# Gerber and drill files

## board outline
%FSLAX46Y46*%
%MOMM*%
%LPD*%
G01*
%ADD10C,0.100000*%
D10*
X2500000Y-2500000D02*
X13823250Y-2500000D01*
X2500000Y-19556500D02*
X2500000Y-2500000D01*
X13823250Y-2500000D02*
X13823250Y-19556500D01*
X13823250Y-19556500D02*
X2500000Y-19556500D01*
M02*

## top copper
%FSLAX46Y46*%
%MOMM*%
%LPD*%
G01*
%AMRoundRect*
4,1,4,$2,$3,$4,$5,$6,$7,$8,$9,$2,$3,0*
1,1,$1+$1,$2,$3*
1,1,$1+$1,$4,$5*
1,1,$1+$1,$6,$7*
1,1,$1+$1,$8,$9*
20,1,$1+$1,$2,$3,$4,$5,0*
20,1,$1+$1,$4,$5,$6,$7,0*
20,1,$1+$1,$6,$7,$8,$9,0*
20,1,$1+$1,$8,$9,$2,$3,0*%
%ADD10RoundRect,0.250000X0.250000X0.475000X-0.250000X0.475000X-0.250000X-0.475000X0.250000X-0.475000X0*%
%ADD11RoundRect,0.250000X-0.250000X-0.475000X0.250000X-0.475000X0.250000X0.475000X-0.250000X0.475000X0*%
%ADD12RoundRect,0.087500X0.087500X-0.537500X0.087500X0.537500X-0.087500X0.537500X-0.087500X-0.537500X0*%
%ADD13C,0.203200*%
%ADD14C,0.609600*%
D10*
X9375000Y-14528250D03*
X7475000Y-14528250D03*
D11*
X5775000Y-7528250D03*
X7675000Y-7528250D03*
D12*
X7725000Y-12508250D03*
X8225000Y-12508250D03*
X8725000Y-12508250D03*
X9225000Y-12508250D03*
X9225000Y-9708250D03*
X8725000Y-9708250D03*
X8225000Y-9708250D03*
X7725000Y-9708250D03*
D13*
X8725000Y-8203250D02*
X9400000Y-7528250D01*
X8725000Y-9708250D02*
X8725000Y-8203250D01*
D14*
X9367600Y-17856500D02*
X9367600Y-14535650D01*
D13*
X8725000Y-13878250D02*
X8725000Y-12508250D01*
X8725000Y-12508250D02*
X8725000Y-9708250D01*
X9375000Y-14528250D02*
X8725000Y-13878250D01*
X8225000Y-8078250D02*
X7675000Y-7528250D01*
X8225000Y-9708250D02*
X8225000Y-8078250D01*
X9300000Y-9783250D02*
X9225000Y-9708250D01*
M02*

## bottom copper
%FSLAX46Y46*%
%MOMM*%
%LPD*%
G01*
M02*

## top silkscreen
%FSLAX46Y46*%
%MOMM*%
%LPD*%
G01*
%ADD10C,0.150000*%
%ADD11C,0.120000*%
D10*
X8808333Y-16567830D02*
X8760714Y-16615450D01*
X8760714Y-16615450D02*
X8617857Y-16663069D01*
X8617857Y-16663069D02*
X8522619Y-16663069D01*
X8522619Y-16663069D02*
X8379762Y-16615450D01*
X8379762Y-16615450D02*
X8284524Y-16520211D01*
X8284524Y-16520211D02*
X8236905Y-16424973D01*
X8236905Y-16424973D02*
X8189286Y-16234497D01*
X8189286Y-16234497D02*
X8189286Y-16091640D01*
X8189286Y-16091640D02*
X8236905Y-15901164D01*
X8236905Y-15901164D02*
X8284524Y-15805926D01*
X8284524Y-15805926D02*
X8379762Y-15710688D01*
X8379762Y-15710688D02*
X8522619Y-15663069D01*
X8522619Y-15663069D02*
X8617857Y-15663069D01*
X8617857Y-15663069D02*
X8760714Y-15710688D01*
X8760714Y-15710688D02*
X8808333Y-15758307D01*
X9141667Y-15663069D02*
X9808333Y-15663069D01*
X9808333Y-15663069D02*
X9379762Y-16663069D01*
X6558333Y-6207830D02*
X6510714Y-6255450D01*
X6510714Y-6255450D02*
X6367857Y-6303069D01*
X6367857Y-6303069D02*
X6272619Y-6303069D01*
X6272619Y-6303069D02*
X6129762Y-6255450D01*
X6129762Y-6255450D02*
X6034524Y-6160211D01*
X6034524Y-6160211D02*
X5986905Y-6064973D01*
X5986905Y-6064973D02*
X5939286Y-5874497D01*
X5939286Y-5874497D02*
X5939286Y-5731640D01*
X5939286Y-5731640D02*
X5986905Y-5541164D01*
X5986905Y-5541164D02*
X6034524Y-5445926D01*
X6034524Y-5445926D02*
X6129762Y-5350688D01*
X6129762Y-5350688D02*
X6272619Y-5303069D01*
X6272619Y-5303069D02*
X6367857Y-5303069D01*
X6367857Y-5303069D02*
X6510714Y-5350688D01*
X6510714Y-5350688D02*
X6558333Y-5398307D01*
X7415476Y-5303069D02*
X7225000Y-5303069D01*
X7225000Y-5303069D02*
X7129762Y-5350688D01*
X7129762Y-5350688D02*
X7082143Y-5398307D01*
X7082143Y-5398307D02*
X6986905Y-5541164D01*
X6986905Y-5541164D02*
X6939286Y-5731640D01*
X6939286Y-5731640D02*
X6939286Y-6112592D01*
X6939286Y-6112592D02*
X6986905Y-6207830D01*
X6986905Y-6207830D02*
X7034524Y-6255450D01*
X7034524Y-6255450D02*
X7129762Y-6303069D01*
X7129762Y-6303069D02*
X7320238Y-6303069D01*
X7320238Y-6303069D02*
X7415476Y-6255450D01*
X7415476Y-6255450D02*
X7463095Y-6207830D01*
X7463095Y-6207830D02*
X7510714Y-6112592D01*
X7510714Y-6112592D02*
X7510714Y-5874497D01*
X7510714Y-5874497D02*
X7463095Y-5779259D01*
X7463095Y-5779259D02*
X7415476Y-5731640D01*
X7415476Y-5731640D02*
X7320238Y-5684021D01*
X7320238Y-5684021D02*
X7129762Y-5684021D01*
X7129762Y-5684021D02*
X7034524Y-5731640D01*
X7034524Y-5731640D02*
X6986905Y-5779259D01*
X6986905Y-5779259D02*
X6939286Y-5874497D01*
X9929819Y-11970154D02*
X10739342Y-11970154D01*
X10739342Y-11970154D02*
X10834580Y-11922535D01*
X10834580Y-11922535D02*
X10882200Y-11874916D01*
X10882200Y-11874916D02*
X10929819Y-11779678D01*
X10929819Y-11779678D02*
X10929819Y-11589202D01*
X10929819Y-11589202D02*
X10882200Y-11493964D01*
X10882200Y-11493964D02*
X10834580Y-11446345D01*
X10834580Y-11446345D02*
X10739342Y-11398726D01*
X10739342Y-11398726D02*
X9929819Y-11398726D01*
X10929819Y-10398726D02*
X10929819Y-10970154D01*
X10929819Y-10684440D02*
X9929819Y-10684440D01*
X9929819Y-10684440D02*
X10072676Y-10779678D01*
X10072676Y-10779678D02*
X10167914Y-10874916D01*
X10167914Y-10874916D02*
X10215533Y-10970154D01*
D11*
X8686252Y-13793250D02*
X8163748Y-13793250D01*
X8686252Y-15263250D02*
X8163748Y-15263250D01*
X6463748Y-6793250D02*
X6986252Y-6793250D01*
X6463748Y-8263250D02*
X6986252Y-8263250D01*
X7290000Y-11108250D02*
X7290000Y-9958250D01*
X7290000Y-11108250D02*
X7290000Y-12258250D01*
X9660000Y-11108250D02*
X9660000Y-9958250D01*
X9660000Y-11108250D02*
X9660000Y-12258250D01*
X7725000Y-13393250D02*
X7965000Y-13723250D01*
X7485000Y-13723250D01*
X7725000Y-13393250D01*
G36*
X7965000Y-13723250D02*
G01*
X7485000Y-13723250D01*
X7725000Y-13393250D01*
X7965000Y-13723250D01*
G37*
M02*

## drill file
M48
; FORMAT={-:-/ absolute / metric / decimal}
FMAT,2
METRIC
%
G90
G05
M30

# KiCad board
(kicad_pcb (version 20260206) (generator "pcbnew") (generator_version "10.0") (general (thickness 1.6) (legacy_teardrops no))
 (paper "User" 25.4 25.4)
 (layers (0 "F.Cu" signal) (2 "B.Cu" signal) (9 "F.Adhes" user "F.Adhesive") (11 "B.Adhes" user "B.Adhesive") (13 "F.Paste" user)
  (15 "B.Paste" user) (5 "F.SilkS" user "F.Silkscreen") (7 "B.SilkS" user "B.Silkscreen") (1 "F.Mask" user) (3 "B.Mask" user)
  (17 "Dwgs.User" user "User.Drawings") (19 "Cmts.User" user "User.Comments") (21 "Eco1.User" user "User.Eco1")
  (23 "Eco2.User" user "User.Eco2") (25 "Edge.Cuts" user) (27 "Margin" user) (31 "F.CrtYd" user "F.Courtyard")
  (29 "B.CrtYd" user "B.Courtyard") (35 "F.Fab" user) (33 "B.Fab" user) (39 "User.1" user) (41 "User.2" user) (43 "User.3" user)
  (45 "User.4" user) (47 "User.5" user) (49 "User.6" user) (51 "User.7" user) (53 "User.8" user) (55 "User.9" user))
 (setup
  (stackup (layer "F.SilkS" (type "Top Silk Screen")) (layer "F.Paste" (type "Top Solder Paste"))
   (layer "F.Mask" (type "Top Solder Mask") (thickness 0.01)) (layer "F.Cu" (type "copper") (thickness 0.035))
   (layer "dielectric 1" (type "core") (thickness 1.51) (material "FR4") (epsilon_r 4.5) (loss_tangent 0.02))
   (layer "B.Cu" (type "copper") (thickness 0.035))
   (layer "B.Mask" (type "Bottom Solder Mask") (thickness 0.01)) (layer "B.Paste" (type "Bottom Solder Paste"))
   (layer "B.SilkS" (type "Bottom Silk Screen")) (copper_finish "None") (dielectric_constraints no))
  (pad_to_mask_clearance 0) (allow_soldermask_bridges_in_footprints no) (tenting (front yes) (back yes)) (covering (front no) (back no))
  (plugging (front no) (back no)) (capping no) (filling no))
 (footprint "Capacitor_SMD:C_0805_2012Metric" (layer "F.Cu") (at 8.425 14.52825 180)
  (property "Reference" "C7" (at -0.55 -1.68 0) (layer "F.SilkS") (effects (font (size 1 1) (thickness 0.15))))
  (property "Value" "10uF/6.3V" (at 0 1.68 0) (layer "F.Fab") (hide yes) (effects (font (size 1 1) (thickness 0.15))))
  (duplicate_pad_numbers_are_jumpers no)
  (fp_line (start -0.261252 0.735) (end 0.261252 0.735) (stroke (width 0.12) (type solid)) (layer "F.SilkS"))
  (fp_line (start -0.261252 -0.735) (end 0.261252 -0.735) (stroke (width 0.12) (type solid)) (layer "F.SilkS"))
  (pad "1" smd roundrect (at -0.95 0 180) (size 1 1.45) (layers "F.Cu" "F.Mask" "F.Paste") (roundrect_rratio 0.25) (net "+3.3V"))
  (pad "2" smd roundrect (at 0.95 0 180) (size 1 1.45) (layers "F.Cu" "F.Mask" "F.Paste") (roundrect_rratio 0.25) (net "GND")))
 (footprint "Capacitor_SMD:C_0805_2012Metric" (layer "F.Cu") (at 6.725 7.52825)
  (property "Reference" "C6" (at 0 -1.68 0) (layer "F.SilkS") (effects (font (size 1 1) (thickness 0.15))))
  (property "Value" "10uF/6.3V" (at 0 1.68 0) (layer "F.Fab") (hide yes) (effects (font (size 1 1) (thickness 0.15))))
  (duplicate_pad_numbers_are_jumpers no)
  (fp_line (start -0.261252 -0.735) (end 0.261252 -0.735) (stroke (width 0.12) (type solid)) (layer "F.SilkS"))
  (fp_line (start -0.261252 0.735) (end 0.261252 0.735) (stroke (width 0.12) (type solid)) (layer "F.SilkS"))
  (pad "1" smd roundrect (at -0.95 0) (size 1 1.45) (layers "F.Cu" "F.Mask" "F.Paste") (roundrect_rratio 0.25) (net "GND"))
  (pad "2" smd roundrect (at 0.95 0) (size 1 1.45) (layers "F.Cu" "F.Mask" "F.Paste") (roundrect_rratio 0.25) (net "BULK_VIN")))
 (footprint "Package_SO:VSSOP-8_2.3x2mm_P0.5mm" (layer "F.Cu") (at 8.475 11.10825 90)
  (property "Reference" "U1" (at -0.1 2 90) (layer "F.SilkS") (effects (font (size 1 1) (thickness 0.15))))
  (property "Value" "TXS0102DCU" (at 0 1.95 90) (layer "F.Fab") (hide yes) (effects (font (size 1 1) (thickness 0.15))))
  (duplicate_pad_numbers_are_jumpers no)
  (fp_line (start 0 -1.185) (end 1.15 -1.185) (stroke (width 0.12) (type solid)) (layer "F.SilkS"))
  (fp_line (start 0 -1.185) (end -1.15 -1.185) (stroke (width 0.12) (type solid)) (layer "F.SilkS"))
  (fp_line (start 0 1.185) (end 1.15 1.185) (stroke (width 0.12) (type solid)) (layer "F.SilkS"))
  (fp_line (start 0 1.185) (end -1.15 1.185) (stroke (width 0.12) (type solid)) (layer "F.SilkS"))
  (fp_poly (pts (xy -2.285 -0.75) (xy -2.615 -0.51) (xy -2.615 -0.99)) (stroke (width 0.12) (type solid)) (fill yes) (layer "F.SilkS"))
  (pad "1" smd roundrect (at -1.4 -0.75 90) (size 1.25 0.35) (layers "F.Cu" "F.Mask" "F.Paste") (roundrect_rratio 0.25) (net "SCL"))
  (pad "2" smd roundrect (at -1.4 -0.25 90) (size 1.25 0.35) (layers "F.Cu" "F.Mask" "F.Paste") (roundrect_rratio 0.25) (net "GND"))
  (pad "3" smd roundrect (at -1.4 0.25 90) (size 1.25 0.35) (layers "F.Cu" "F.Mask" "F.Paste") (roundrect_rratio 0.25) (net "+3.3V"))
  (pad "4" smd roundrect (at -1.4 0.75 90) (size 1.25 0.35) (layers "F.Cu" "F.Mask" "F.Paste") (roundrect_rratio 0.25) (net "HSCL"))
  (pad "5" smd roundrect (at 1.4 0.75 90) (size 1.25 0.35) (layers "F.Cu" "F.Mask" "F.Paste") (roundrect_rratio 0.25) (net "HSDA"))
  (pad "6" smd roundrect (at 1.4 0.25 90) (size 1.25 0.35) (layers "F.Cu" "F.Mask" "F.Paste") (roundrect_rratio 0.25) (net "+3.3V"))
  (pad "7" smd roundrect (at 1.4 -0.25 90) (size 1.25 0.35) (layers "F.Cu" "F.Mask" "F.Paste") (roundrect_rratio 0.25) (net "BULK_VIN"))
  (pad "8" smd roundrect (at 1.4 -0.75 90) (size 1.25 0.35) (layers "F.Cu" "F.Mask" "F.Paste") (roundrect_rratio 0.25) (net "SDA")))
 (gr_line (start 2.5 2.5) (end 13.82325 2.5) (stroke (width 0.1) (type default)) (layer "Edge.Cuts"))
 (gr_line (start 2.5 19.5565) (end 2.5 2.5) (stroke (width 0.1) (type default)) (layer "Edge.Cuts"))
 (gr_line (start 13.82325 2.5) (end 13.82325 19.5565) (stroke (width 0.1) (type default)) (layer "Edge.Cuts"))
 (gr_line (start 13.82325 19.5565) (end 2.5 19.5565) (stroke (width 0.1) (type default)) (layer "Edge.Cuts"))
 (segment (start 8.725 8.20325) (end 9.4 7.52825) (width 0.2032) (layer "F.Cu") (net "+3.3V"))
 (segment (start 8.725 9.70825) (end 8.725 8.20325) (width 0.2032) (layer "F.Cu") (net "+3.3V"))
 (segment (start 9.3676 17.8565) (end 9.3676 14.53565) (width 0.6096) (layer "F.Cu") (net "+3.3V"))
 (segment (start 8.725 13.87825) (end 8.725 12.50825) (width 0.2032) (layer "F.Cu") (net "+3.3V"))
 (segment (start 8.725 12.50825) (end 8.725 9.70825) (width 0.2032) (layer "F.Cu") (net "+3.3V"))
 (segment (start 9.375 14.52825) (end 8.725 13.87825) (width 0.2032) (layer "F.Cu") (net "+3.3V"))
 (segment (start 8.225 8.07825) (end 7.675 7.52825) (width 0.2032) (layer "F.Cu") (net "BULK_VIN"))
 (segment (start 8.225 9.70825) (end 8.225 8.07825) (width 0.2032) (layer "F.Cu") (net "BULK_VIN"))
 (segment (start 9.3 9.78325) (end 9.225 9.70825) (width 0.2032) (layer "F.Cu") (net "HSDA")))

